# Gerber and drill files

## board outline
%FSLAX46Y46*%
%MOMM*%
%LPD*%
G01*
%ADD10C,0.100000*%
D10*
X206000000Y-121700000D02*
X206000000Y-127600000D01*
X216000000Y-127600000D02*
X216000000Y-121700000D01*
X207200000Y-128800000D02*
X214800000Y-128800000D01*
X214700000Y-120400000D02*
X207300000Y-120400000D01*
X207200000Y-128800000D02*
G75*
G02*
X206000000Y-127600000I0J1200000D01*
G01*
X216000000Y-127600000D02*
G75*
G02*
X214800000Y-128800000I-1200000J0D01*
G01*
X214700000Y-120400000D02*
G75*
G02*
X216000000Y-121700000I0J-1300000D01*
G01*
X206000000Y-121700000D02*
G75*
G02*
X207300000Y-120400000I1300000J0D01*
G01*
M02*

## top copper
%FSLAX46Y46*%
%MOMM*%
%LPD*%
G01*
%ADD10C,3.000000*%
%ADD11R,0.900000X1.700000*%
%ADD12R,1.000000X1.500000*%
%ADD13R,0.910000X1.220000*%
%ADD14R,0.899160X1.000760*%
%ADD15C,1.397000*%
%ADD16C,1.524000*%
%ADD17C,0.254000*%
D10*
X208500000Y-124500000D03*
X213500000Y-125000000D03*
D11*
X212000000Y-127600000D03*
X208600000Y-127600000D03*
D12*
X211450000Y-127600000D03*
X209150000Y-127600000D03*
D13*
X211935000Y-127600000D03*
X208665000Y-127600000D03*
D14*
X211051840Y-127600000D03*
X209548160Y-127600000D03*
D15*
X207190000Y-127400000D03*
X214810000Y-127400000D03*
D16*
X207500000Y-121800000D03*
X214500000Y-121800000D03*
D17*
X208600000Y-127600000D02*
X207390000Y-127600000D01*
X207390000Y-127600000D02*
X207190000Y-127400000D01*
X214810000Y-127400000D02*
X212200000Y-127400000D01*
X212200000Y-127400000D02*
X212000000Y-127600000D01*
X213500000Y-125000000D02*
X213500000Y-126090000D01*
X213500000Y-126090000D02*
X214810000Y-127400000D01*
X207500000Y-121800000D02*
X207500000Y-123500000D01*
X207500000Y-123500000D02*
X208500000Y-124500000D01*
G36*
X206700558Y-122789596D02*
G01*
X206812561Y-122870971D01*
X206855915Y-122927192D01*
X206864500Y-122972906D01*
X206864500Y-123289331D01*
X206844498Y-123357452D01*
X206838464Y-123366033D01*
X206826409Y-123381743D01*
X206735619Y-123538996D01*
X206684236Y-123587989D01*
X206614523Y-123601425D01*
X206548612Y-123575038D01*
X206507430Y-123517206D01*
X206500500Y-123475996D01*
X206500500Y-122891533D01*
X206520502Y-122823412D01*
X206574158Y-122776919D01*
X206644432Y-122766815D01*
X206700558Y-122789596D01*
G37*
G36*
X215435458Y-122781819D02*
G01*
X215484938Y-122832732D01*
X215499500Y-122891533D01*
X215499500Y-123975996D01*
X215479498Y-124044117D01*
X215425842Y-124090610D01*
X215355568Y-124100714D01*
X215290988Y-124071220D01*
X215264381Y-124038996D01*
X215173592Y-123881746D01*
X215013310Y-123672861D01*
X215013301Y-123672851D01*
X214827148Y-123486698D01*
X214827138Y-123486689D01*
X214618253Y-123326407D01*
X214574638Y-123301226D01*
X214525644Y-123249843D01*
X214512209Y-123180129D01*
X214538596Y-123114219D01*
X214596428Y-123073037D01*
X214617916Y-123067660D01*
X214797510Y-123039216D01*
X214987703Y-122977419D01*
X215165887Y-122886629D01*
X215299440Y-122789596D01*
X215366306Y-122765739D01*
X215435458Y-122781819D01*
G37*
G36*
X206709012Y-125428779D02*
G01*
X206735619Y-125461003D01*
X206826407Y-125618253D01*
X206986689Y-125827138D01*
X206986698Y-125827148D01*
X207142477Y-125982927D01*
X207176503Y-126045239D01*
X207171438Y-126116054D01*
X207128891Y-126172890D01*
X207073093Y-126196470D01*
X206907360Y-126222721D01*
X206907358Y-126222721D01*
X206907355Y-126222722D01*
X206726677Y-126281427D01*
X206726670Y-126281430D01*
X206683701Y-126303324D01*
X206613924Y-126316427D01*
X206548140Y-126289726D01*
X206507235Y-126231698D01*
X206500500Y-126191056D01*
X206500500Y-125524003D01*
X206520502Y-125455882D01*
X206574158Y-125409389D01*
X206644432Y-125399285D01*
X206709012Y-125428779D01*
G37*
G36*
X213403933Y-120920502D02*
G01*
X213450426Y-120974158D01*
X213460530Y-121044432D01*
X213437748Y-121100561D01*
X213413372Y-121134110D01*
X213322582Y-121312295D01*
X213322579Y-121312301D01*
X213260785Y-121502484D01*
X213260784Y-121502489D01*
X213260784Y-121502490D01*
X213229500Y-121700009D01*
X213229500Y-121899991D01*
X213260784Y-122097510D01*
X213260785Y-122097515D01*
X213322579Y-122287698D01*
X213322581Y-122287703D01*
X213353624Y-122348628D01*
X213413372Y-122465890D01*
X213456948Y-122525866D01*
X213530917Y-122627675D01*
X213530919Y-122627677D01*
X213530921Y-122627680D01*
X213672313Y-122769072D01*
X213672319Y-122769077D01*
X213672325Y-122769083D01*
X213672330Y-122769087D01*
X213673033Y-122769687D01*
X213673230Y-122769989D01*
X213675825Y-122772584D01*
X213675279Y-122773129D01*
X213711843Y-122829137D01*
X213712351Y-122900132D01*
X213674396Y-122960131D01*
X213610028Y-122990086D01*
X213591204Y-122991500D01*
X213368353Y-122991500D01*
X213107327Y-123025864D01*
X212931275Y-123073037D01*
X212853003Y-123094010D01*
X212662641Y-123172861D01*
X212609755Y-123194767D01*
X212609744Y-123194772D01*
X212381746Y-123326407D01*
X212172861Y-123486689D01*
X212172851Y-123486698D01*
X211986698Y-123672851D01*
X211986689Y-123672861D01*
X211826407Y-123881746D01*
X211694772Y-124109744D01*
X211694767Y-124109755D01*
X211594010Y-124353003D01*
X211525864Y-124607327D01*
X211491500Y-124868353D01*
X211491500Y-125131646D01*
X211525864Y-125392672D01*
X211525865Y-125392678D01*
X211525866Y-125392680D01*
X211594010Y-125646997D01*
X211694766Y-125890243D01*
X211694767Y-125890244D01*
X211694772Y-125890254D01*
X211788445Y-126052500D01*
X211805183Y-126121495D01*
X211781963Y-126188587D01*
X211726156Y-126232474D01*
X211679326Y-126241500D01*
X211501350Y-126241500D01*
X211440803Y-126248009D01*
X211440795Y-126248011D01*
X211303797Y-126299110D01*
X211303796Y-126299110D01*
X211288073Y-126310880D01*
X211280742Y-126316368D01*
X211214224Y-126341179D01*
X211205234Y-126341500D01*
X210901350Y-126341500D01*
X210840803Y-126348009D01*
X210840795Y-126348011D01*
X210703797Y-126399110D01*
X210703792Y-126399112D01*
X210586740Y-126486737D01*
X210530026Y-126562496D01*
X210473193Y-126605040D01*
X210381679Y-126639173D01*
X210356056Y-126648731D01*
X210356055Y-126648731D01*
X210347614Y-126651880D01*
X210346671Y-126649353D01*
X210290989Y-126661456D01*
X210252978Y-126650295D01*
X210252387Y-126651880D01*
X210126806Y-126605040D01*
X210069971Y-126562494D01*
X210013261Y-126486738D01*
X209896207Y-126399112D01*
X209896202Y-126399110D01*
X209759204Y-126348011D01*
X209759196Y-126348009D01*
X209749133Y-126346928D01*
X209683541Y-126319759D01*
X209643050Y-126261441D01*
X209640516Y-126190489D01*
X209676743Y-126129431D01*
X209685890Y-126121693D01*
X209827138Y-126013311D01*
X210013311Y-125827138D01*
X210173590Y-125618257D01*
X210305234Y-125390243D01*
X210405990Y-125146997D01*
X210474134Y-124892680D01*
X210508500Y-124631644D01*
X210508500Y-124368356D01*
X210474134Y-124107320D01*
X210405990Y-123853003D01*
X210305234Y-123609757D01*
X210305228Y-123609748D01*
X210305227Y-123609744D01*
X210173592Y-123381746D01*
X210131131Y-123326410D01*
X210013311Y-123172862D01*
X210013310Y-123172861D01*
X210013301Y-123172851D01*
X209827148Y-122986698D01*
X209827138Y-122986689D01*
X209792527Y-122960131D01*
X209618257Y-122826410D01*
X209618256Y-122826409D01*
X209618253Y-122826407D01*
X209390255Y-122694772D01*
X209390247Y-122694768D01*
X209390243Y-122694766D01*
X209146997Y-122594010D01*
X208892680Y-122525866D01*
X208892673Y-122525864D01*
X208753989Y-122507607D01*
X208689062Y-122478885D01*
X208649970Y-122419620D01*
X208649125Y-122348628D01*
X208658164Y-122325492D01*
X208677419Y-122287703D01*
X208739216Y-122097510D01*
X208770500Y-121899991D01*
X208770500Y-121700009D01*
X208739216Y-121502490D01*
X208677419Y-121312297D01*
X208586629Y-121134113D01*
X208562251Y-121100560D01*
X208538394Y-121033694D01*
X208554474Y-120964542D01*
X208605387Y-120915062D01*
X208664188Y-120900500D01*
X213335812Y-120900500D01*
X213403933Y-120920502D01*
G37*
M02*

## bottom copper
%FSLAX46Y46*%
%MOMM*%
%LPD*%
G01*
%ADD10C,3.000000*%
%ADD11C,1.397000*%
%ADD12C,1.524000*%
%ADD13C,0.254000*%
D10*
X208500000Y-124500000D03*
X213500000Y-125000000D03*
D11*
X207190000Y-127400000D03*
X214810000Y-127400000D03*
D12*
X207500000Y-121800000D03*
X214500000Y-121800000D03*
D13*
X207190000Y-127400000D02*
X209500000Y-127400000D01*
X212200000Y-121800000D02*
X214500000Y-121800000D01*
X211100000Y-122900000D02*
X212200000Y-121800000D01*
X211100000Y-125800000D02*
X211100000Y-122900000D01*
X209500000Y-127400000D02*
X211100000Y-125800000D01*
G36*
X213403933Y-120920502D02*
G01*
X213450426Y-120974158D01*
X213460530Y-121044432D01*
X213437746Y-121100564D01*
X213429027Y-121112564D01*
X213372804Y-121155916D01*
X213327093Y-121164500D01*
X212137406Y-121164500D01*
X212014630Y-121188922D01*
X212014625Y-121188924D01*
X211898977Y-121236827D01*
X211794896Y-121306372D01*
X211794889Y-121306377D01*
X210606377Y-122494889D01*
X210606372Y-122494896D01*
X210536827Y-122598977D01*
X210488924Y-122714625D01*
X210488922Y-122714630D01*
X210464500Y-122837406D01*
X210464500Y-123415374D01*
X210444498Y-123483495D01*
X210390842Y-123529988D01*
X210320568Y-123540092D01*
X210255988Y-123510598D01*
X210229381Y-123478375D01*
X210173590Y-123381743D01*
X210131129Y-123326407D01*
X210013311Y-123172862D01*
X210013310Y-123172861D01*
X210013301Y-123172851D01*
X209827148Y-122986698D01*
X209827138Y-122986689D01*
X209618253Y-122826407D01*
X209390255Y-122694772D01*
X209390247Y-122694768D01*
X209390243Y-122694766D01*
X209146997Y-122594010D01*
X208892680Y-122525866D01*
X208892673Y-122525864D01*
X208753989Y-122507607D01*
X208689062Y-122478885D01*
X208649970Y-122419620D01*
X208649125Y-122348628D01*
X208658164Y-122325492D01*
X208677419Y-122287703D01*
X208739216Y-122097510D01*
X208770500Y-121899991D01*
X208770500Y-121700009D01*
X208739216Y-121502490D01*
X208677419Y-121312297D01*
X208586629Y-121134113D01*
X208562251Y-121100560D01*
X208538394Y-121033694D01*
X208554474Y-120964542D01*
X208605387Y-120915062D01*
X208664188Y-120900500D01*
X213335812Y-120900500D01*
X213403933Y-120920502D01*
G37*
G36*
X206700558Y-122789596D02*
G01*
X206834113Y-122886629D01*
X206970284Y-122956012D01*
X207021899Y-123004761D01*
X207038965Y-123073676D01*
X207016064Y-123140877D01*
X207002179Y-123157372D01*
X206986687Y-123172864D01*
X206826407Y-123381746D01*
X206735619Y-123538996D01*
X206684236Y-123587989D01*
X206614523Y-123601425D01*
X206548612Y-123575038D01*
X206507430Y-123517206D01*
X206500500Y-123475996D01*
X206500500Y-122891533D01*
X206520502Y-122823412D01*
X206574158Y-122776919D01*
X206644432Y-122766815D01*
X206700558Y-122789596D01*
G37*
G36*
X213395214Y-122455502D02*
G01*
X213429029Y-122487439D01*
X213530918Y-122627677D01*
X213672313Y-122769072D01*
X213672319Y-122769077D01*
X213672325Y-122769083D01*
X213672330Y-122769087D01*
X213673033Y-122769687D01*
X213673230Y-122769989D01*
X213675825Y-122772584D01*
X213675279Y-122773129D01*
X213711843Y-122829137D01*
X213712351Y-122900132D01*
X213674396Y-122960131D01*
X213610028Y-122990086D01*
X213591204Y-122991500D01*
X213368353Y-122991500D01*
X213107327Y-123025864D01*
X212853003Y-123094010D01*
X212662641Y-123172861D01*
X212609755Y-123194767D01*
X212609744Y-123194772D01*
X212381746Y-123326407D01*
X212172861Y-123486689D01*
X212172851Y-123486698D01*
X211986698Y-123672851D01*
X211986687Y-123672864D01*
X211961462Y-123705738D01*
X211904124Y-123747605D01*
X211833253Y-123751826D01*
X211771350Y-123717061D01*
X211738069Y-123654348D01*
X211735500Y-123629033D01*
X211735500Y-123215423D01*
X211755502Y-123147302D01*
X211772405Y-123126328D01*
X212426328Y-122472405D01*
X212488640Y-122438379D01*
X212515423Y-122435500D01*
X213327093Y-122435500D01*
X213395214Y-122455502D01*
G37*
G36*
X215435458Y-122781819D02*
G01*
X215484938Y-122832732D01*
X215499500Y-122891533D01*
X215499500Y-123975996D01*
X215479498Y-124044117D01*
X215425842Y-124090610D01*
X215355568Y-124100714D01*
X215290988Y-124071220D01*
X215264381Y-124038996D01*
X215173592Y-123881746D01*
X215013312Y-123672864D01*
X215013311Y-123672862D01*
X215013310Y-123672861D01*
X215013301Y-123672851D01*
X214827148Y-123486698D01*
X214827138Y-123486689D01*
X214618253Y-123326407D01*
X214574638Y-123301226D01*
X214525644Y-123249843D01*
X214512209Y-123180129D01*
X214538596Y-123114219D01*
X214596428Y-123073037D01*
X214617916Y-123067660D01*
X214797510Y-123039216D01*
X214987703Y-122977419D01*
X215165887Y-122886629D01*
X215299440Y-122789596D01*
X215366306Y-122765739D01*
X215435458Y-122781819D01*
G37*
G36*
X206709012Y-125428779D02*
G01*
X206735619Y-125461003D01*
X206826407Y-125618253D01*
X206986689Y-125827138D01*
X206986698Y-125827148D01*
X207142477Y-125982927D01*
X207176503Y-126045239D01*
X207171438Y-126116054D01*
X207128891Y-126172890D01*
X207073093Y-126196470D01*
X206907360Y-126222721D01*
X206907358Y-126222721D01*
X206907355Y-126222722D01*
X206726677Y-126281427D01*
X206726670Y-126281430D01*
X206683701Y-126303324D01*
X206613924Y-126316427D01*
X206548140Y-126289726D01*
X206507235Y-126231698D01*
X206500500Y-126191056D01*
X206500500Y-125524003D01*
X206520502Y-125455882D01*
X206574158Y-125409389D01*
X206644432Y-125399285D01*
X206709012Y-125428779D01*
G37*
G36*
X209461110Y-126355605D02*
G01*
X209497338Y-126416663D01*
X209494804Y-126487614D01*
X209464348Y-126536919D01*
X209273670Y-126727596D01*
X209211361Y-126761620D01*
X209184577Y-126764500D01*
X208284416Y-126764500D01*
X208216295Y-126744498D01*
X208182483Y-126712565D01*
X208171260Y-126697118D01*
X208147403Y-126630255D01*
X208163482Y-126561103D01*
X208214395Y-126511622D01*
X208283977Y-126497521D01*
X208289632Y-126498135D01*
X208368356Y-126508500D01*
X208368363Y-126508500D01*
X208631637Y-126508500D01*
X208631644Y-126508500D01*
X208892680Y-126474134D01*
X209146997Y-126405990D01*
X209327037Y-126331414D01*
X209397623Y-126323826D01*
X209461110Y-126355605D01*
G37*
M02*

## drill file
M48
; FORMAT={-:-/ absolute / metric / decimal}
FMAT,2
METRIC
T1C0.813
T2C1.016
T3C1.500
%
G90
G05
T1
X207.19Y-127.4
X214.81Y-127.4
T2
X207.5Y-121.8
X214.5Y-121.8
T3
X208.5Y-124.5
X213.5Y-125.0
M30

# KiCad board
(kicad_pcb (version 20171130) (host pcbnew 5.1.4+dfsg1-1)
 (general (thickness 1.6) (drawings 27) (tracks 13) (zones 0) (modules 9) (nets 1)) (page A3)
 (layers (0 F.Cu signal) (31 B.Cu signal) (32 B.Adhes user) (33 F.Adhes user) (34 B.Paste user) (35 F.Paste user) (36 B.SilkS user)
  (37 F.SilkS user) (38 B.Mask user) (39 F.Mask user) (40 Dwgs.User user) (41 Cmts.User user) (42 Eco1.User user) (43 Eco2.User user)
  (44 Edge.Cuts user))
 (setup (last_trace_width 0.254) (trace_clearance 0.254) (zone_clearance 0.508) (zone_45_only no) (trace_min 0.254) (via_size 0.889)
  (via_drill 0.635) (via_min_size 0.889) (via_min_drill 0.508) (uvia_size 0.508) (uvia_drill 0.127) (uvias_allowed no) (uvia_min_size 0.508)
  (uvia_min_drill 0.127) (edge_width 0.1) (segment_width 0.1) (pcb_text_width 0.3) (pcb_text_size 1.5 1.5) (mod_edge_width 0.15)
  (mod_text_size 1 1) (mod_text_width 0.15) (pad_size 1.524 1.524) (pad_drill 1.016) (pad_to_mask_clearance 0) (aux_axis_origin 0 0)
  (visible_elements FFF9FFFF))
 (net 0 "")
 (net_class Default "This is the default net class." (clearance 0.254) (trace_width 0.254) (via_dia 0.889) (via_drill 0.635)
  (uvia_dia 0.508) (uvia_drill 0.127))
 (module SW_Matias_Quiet (layer F.Cu) (at 211 129)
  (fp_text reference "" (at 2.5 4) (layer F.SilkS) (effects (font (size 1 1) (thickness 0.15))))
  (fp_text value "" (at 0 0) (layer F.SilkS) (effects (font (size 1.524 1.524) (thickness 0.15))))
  (pad 1 thru_hole circle (at -2.5 -4.5) (size 3 3) (drill 1.5) (layers *.Cu *.Mask F.SilkS))
  (pad 2 thru_hole circle (at 2.5 -4) (size 3 3) (drill 1.5) (layers *.Cu *.Mask F.SilkS)))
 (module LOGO (layer F.Cu) (at 211.1 123.1)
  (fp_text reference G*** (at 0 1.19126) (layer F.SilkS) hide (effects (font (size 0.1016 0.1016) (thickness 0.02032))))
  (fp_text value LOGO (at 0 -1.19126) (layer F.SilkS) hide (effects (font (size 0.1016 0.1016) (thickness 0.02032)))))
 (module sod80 (layer F.Cu) (at 210.3 127.6)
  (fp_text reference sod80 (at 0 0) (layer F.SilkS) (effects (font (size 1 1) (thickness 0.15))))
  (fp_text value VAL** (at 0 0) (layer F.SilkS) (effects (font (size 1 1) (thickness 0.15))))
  (pad 5 smd rect (at 1.7 0) (size 0.9 1.7) (layers F.Cu F.Paste F.Mask))
  (pad 6 smd rect (at -1.7 0) (size 0.9 1.7) (layers F.Cu F.Paste F.Mask)))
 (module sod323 (layer F.Cu) (at 210.3 127.6)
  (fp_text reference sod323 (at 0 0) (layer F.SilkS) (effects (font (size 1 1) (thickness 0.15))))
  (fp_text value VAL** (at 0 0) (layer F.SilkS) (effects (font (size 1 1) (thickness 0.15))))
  (pad 3 smd rect (at 1.15 0) (size 1 1.5) (layers F.Cu F.Paste F.Mask))
  (pad 4 smd rect (at -1.15 0) (size 1 1.5) (layers F.Cu F.Paste F.Mask)))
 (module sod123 (layer F.Cu) (at 210.3 127.6)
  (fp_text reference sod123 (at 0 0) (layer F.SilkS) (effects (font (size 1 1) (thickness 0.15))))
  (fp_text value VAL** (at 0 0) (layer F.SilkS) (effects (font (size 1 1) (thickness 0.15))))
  (pad 1 smd rect (at 1.635 0) (size 0.91 1.22) (layers F.Cu F.Paste F.Mask))
  (pad 2 smd rect (at -1.635 0) (size 0.91 1.22) (layers F.Cu F.Paste F.Mask)))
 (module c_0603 (layer F.Cu) (at 210.3 127.6)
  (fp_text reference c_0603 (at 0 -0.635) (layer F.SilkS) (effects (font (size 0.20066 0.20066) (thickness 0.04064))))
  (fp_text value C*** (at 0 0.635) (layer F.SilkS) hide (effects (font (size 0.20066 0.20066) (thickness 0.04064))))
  (pad 1 smd rect (at 0.75184 0) (size 0.89916 1.00076) (layers F.Cu F.Paste F.Mask))
  (pad 2 smd rect (at -0.75184 0) (size 0.89916 1.00076) (layers F.Cu F.Paste F.Mask)))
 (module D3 (layer F.Cu) (at 211 127.4 180)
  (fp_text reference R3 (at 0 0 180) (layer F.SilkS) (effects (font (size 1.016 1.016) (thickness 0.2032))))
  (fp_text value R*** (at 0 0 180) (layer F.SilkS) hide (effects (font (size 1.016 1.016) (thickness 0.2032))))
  (pad 2 thru_hole circle (at 3.81 0 180) (size 1.397 1.397) (drill 0.8128) (layers *.Cu *.Mask F.SilkS))
  (pad 1 thru_hole circle (at -3.81 0 180) (size 1.397 1.397) (drill 0.8128) (layers *.Cu *.Mask F.SilkS)))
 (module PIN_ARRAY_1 (layer F.Cu) (at 207.5 121.8)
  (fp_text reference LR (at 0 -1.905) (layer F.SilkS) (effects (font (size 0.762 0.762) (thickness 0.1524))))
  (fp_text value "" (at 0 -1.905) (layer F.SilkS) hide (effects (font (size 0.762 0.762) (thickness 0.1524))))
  (pad 1 thru_hole circle (at 0 0) (size 1.524 1.524) (drill 1.016) (layers *.Cu *.Mask F.SilkS)))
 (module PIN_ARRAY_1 (layer F.Cu) (at 214.5 121.8)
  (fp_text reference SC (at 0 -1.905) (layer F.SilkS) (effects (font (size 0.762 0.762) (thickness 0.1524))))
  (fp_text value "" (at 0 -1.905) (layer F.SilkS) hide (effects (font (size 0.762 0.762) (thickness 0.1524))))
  (pad 1 thru_hole circle (at 0 0) (size 1.524 1.524) (drill 1.016) (layers *.Cu *.Mask F.SilkS)))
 (gr_line (start 206 121.7) (end 206 127.6) (angle 90) (layer Edge.Cuts) (width 0.1))
 (gr_line (start 216 127.6) (end 216 121.7) (angle 90) (layer Edge.Cuts) (width 0.1))
 (gr_line (start 207.2 128.8) (end 214.8 128.8) (angle 90) (layer Edge.Cuts) (width 0.1))
 (gr_line (start 214.7 120.4) (end 207.3 120.4) (angle 90) (layer Edge.Cuts) (width 0.1))
 (gr_arc (start 207.2 127.6) (end 207.2 128.8) (angle 90) (layer Edge.Cuts) (width 0.1))
 (gr_arc (start 214.8 127.6) (end 216 127.6) (angle 90) (layer Edge.Cuts) (width 0.1))
 (gr_arc (start 214.7 121.7) (end 214.7 120.4) (angle 90) (layer Edge.Cuts) (width 0.1))
 (gr_arc (start 207.3 121.7) (end 206 121.7) (angle 90) (layer Edge.Cuts) (width 0.1))
 (segment (start 207.19 127.4) (end 209.5 127.4) (width 0.254) (layer B.Cu) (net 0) (status 400000))
 (segment (start 212.2 121.8) (end 214.5 121.8) (width 0.254) (layer B.Cu) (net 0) (status 800000))
 (segment (start 211.1 122.9) (end 212.2 121.8) (width 0.254) (layer B.Cu) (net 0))
 (segment (start 211.1 125.8) (end 211.1 122.9) (width 0.254) (layer B.Cu) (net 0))
 (segment (start 209.5 127.4) (end 211.1 125.8) (width 0.254) (layer B.Cu) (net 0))
 (segment (start 208.6 127.6) (end 207.39 127.6) (width 0.254) (layer F.Cu) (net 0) (status C00000))
 (segment (start 207.39 127.6) (end 207.19 127.4) (width 0.254) (layer F.Cu) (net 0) (status C00000))
 (segment (start 214.81 127.4) (end 212.2 127.4) (width 0.254) (layer F.Cu) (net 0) (status C00000))
 (segment (start 212.2 127.4) (end 212 127.6) (width 0.254) (layer F.Cu) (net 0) (status C00000))
 (segment (start 213.5 125) (end 213.5 126.09) (width 0.254) (layer F.Cu) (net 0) (status C00000))
 (segment (start 213.5 126.09) (end 214.81 127.4) (width 0.254) (layer F.Cu) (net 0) (status C00000))
 (segment (start 207.5 121.8) (end 207.5 123.5) (width 0.254) (layer F.Cu) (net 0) (status C00000))
 (segment (start 207.5 123.5) (end 208.5 124.5) (width 0.254) (layer F.Cu) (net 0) (status C00000))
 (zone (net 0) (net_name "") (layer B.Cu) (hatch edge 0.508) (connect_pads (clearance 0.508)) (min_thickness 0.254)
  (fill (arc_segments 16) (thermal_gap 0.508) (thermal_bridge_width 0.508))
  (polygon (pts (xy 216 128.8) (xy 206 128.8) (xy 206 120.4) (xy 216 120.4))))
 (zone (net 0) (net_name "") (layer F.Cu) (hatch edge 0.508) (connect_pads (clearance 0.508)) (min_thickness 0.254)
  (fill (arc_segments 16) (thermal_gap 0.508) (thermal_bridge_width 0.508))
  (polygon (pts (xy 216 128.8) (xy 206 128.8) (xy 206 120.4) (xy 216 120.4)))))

